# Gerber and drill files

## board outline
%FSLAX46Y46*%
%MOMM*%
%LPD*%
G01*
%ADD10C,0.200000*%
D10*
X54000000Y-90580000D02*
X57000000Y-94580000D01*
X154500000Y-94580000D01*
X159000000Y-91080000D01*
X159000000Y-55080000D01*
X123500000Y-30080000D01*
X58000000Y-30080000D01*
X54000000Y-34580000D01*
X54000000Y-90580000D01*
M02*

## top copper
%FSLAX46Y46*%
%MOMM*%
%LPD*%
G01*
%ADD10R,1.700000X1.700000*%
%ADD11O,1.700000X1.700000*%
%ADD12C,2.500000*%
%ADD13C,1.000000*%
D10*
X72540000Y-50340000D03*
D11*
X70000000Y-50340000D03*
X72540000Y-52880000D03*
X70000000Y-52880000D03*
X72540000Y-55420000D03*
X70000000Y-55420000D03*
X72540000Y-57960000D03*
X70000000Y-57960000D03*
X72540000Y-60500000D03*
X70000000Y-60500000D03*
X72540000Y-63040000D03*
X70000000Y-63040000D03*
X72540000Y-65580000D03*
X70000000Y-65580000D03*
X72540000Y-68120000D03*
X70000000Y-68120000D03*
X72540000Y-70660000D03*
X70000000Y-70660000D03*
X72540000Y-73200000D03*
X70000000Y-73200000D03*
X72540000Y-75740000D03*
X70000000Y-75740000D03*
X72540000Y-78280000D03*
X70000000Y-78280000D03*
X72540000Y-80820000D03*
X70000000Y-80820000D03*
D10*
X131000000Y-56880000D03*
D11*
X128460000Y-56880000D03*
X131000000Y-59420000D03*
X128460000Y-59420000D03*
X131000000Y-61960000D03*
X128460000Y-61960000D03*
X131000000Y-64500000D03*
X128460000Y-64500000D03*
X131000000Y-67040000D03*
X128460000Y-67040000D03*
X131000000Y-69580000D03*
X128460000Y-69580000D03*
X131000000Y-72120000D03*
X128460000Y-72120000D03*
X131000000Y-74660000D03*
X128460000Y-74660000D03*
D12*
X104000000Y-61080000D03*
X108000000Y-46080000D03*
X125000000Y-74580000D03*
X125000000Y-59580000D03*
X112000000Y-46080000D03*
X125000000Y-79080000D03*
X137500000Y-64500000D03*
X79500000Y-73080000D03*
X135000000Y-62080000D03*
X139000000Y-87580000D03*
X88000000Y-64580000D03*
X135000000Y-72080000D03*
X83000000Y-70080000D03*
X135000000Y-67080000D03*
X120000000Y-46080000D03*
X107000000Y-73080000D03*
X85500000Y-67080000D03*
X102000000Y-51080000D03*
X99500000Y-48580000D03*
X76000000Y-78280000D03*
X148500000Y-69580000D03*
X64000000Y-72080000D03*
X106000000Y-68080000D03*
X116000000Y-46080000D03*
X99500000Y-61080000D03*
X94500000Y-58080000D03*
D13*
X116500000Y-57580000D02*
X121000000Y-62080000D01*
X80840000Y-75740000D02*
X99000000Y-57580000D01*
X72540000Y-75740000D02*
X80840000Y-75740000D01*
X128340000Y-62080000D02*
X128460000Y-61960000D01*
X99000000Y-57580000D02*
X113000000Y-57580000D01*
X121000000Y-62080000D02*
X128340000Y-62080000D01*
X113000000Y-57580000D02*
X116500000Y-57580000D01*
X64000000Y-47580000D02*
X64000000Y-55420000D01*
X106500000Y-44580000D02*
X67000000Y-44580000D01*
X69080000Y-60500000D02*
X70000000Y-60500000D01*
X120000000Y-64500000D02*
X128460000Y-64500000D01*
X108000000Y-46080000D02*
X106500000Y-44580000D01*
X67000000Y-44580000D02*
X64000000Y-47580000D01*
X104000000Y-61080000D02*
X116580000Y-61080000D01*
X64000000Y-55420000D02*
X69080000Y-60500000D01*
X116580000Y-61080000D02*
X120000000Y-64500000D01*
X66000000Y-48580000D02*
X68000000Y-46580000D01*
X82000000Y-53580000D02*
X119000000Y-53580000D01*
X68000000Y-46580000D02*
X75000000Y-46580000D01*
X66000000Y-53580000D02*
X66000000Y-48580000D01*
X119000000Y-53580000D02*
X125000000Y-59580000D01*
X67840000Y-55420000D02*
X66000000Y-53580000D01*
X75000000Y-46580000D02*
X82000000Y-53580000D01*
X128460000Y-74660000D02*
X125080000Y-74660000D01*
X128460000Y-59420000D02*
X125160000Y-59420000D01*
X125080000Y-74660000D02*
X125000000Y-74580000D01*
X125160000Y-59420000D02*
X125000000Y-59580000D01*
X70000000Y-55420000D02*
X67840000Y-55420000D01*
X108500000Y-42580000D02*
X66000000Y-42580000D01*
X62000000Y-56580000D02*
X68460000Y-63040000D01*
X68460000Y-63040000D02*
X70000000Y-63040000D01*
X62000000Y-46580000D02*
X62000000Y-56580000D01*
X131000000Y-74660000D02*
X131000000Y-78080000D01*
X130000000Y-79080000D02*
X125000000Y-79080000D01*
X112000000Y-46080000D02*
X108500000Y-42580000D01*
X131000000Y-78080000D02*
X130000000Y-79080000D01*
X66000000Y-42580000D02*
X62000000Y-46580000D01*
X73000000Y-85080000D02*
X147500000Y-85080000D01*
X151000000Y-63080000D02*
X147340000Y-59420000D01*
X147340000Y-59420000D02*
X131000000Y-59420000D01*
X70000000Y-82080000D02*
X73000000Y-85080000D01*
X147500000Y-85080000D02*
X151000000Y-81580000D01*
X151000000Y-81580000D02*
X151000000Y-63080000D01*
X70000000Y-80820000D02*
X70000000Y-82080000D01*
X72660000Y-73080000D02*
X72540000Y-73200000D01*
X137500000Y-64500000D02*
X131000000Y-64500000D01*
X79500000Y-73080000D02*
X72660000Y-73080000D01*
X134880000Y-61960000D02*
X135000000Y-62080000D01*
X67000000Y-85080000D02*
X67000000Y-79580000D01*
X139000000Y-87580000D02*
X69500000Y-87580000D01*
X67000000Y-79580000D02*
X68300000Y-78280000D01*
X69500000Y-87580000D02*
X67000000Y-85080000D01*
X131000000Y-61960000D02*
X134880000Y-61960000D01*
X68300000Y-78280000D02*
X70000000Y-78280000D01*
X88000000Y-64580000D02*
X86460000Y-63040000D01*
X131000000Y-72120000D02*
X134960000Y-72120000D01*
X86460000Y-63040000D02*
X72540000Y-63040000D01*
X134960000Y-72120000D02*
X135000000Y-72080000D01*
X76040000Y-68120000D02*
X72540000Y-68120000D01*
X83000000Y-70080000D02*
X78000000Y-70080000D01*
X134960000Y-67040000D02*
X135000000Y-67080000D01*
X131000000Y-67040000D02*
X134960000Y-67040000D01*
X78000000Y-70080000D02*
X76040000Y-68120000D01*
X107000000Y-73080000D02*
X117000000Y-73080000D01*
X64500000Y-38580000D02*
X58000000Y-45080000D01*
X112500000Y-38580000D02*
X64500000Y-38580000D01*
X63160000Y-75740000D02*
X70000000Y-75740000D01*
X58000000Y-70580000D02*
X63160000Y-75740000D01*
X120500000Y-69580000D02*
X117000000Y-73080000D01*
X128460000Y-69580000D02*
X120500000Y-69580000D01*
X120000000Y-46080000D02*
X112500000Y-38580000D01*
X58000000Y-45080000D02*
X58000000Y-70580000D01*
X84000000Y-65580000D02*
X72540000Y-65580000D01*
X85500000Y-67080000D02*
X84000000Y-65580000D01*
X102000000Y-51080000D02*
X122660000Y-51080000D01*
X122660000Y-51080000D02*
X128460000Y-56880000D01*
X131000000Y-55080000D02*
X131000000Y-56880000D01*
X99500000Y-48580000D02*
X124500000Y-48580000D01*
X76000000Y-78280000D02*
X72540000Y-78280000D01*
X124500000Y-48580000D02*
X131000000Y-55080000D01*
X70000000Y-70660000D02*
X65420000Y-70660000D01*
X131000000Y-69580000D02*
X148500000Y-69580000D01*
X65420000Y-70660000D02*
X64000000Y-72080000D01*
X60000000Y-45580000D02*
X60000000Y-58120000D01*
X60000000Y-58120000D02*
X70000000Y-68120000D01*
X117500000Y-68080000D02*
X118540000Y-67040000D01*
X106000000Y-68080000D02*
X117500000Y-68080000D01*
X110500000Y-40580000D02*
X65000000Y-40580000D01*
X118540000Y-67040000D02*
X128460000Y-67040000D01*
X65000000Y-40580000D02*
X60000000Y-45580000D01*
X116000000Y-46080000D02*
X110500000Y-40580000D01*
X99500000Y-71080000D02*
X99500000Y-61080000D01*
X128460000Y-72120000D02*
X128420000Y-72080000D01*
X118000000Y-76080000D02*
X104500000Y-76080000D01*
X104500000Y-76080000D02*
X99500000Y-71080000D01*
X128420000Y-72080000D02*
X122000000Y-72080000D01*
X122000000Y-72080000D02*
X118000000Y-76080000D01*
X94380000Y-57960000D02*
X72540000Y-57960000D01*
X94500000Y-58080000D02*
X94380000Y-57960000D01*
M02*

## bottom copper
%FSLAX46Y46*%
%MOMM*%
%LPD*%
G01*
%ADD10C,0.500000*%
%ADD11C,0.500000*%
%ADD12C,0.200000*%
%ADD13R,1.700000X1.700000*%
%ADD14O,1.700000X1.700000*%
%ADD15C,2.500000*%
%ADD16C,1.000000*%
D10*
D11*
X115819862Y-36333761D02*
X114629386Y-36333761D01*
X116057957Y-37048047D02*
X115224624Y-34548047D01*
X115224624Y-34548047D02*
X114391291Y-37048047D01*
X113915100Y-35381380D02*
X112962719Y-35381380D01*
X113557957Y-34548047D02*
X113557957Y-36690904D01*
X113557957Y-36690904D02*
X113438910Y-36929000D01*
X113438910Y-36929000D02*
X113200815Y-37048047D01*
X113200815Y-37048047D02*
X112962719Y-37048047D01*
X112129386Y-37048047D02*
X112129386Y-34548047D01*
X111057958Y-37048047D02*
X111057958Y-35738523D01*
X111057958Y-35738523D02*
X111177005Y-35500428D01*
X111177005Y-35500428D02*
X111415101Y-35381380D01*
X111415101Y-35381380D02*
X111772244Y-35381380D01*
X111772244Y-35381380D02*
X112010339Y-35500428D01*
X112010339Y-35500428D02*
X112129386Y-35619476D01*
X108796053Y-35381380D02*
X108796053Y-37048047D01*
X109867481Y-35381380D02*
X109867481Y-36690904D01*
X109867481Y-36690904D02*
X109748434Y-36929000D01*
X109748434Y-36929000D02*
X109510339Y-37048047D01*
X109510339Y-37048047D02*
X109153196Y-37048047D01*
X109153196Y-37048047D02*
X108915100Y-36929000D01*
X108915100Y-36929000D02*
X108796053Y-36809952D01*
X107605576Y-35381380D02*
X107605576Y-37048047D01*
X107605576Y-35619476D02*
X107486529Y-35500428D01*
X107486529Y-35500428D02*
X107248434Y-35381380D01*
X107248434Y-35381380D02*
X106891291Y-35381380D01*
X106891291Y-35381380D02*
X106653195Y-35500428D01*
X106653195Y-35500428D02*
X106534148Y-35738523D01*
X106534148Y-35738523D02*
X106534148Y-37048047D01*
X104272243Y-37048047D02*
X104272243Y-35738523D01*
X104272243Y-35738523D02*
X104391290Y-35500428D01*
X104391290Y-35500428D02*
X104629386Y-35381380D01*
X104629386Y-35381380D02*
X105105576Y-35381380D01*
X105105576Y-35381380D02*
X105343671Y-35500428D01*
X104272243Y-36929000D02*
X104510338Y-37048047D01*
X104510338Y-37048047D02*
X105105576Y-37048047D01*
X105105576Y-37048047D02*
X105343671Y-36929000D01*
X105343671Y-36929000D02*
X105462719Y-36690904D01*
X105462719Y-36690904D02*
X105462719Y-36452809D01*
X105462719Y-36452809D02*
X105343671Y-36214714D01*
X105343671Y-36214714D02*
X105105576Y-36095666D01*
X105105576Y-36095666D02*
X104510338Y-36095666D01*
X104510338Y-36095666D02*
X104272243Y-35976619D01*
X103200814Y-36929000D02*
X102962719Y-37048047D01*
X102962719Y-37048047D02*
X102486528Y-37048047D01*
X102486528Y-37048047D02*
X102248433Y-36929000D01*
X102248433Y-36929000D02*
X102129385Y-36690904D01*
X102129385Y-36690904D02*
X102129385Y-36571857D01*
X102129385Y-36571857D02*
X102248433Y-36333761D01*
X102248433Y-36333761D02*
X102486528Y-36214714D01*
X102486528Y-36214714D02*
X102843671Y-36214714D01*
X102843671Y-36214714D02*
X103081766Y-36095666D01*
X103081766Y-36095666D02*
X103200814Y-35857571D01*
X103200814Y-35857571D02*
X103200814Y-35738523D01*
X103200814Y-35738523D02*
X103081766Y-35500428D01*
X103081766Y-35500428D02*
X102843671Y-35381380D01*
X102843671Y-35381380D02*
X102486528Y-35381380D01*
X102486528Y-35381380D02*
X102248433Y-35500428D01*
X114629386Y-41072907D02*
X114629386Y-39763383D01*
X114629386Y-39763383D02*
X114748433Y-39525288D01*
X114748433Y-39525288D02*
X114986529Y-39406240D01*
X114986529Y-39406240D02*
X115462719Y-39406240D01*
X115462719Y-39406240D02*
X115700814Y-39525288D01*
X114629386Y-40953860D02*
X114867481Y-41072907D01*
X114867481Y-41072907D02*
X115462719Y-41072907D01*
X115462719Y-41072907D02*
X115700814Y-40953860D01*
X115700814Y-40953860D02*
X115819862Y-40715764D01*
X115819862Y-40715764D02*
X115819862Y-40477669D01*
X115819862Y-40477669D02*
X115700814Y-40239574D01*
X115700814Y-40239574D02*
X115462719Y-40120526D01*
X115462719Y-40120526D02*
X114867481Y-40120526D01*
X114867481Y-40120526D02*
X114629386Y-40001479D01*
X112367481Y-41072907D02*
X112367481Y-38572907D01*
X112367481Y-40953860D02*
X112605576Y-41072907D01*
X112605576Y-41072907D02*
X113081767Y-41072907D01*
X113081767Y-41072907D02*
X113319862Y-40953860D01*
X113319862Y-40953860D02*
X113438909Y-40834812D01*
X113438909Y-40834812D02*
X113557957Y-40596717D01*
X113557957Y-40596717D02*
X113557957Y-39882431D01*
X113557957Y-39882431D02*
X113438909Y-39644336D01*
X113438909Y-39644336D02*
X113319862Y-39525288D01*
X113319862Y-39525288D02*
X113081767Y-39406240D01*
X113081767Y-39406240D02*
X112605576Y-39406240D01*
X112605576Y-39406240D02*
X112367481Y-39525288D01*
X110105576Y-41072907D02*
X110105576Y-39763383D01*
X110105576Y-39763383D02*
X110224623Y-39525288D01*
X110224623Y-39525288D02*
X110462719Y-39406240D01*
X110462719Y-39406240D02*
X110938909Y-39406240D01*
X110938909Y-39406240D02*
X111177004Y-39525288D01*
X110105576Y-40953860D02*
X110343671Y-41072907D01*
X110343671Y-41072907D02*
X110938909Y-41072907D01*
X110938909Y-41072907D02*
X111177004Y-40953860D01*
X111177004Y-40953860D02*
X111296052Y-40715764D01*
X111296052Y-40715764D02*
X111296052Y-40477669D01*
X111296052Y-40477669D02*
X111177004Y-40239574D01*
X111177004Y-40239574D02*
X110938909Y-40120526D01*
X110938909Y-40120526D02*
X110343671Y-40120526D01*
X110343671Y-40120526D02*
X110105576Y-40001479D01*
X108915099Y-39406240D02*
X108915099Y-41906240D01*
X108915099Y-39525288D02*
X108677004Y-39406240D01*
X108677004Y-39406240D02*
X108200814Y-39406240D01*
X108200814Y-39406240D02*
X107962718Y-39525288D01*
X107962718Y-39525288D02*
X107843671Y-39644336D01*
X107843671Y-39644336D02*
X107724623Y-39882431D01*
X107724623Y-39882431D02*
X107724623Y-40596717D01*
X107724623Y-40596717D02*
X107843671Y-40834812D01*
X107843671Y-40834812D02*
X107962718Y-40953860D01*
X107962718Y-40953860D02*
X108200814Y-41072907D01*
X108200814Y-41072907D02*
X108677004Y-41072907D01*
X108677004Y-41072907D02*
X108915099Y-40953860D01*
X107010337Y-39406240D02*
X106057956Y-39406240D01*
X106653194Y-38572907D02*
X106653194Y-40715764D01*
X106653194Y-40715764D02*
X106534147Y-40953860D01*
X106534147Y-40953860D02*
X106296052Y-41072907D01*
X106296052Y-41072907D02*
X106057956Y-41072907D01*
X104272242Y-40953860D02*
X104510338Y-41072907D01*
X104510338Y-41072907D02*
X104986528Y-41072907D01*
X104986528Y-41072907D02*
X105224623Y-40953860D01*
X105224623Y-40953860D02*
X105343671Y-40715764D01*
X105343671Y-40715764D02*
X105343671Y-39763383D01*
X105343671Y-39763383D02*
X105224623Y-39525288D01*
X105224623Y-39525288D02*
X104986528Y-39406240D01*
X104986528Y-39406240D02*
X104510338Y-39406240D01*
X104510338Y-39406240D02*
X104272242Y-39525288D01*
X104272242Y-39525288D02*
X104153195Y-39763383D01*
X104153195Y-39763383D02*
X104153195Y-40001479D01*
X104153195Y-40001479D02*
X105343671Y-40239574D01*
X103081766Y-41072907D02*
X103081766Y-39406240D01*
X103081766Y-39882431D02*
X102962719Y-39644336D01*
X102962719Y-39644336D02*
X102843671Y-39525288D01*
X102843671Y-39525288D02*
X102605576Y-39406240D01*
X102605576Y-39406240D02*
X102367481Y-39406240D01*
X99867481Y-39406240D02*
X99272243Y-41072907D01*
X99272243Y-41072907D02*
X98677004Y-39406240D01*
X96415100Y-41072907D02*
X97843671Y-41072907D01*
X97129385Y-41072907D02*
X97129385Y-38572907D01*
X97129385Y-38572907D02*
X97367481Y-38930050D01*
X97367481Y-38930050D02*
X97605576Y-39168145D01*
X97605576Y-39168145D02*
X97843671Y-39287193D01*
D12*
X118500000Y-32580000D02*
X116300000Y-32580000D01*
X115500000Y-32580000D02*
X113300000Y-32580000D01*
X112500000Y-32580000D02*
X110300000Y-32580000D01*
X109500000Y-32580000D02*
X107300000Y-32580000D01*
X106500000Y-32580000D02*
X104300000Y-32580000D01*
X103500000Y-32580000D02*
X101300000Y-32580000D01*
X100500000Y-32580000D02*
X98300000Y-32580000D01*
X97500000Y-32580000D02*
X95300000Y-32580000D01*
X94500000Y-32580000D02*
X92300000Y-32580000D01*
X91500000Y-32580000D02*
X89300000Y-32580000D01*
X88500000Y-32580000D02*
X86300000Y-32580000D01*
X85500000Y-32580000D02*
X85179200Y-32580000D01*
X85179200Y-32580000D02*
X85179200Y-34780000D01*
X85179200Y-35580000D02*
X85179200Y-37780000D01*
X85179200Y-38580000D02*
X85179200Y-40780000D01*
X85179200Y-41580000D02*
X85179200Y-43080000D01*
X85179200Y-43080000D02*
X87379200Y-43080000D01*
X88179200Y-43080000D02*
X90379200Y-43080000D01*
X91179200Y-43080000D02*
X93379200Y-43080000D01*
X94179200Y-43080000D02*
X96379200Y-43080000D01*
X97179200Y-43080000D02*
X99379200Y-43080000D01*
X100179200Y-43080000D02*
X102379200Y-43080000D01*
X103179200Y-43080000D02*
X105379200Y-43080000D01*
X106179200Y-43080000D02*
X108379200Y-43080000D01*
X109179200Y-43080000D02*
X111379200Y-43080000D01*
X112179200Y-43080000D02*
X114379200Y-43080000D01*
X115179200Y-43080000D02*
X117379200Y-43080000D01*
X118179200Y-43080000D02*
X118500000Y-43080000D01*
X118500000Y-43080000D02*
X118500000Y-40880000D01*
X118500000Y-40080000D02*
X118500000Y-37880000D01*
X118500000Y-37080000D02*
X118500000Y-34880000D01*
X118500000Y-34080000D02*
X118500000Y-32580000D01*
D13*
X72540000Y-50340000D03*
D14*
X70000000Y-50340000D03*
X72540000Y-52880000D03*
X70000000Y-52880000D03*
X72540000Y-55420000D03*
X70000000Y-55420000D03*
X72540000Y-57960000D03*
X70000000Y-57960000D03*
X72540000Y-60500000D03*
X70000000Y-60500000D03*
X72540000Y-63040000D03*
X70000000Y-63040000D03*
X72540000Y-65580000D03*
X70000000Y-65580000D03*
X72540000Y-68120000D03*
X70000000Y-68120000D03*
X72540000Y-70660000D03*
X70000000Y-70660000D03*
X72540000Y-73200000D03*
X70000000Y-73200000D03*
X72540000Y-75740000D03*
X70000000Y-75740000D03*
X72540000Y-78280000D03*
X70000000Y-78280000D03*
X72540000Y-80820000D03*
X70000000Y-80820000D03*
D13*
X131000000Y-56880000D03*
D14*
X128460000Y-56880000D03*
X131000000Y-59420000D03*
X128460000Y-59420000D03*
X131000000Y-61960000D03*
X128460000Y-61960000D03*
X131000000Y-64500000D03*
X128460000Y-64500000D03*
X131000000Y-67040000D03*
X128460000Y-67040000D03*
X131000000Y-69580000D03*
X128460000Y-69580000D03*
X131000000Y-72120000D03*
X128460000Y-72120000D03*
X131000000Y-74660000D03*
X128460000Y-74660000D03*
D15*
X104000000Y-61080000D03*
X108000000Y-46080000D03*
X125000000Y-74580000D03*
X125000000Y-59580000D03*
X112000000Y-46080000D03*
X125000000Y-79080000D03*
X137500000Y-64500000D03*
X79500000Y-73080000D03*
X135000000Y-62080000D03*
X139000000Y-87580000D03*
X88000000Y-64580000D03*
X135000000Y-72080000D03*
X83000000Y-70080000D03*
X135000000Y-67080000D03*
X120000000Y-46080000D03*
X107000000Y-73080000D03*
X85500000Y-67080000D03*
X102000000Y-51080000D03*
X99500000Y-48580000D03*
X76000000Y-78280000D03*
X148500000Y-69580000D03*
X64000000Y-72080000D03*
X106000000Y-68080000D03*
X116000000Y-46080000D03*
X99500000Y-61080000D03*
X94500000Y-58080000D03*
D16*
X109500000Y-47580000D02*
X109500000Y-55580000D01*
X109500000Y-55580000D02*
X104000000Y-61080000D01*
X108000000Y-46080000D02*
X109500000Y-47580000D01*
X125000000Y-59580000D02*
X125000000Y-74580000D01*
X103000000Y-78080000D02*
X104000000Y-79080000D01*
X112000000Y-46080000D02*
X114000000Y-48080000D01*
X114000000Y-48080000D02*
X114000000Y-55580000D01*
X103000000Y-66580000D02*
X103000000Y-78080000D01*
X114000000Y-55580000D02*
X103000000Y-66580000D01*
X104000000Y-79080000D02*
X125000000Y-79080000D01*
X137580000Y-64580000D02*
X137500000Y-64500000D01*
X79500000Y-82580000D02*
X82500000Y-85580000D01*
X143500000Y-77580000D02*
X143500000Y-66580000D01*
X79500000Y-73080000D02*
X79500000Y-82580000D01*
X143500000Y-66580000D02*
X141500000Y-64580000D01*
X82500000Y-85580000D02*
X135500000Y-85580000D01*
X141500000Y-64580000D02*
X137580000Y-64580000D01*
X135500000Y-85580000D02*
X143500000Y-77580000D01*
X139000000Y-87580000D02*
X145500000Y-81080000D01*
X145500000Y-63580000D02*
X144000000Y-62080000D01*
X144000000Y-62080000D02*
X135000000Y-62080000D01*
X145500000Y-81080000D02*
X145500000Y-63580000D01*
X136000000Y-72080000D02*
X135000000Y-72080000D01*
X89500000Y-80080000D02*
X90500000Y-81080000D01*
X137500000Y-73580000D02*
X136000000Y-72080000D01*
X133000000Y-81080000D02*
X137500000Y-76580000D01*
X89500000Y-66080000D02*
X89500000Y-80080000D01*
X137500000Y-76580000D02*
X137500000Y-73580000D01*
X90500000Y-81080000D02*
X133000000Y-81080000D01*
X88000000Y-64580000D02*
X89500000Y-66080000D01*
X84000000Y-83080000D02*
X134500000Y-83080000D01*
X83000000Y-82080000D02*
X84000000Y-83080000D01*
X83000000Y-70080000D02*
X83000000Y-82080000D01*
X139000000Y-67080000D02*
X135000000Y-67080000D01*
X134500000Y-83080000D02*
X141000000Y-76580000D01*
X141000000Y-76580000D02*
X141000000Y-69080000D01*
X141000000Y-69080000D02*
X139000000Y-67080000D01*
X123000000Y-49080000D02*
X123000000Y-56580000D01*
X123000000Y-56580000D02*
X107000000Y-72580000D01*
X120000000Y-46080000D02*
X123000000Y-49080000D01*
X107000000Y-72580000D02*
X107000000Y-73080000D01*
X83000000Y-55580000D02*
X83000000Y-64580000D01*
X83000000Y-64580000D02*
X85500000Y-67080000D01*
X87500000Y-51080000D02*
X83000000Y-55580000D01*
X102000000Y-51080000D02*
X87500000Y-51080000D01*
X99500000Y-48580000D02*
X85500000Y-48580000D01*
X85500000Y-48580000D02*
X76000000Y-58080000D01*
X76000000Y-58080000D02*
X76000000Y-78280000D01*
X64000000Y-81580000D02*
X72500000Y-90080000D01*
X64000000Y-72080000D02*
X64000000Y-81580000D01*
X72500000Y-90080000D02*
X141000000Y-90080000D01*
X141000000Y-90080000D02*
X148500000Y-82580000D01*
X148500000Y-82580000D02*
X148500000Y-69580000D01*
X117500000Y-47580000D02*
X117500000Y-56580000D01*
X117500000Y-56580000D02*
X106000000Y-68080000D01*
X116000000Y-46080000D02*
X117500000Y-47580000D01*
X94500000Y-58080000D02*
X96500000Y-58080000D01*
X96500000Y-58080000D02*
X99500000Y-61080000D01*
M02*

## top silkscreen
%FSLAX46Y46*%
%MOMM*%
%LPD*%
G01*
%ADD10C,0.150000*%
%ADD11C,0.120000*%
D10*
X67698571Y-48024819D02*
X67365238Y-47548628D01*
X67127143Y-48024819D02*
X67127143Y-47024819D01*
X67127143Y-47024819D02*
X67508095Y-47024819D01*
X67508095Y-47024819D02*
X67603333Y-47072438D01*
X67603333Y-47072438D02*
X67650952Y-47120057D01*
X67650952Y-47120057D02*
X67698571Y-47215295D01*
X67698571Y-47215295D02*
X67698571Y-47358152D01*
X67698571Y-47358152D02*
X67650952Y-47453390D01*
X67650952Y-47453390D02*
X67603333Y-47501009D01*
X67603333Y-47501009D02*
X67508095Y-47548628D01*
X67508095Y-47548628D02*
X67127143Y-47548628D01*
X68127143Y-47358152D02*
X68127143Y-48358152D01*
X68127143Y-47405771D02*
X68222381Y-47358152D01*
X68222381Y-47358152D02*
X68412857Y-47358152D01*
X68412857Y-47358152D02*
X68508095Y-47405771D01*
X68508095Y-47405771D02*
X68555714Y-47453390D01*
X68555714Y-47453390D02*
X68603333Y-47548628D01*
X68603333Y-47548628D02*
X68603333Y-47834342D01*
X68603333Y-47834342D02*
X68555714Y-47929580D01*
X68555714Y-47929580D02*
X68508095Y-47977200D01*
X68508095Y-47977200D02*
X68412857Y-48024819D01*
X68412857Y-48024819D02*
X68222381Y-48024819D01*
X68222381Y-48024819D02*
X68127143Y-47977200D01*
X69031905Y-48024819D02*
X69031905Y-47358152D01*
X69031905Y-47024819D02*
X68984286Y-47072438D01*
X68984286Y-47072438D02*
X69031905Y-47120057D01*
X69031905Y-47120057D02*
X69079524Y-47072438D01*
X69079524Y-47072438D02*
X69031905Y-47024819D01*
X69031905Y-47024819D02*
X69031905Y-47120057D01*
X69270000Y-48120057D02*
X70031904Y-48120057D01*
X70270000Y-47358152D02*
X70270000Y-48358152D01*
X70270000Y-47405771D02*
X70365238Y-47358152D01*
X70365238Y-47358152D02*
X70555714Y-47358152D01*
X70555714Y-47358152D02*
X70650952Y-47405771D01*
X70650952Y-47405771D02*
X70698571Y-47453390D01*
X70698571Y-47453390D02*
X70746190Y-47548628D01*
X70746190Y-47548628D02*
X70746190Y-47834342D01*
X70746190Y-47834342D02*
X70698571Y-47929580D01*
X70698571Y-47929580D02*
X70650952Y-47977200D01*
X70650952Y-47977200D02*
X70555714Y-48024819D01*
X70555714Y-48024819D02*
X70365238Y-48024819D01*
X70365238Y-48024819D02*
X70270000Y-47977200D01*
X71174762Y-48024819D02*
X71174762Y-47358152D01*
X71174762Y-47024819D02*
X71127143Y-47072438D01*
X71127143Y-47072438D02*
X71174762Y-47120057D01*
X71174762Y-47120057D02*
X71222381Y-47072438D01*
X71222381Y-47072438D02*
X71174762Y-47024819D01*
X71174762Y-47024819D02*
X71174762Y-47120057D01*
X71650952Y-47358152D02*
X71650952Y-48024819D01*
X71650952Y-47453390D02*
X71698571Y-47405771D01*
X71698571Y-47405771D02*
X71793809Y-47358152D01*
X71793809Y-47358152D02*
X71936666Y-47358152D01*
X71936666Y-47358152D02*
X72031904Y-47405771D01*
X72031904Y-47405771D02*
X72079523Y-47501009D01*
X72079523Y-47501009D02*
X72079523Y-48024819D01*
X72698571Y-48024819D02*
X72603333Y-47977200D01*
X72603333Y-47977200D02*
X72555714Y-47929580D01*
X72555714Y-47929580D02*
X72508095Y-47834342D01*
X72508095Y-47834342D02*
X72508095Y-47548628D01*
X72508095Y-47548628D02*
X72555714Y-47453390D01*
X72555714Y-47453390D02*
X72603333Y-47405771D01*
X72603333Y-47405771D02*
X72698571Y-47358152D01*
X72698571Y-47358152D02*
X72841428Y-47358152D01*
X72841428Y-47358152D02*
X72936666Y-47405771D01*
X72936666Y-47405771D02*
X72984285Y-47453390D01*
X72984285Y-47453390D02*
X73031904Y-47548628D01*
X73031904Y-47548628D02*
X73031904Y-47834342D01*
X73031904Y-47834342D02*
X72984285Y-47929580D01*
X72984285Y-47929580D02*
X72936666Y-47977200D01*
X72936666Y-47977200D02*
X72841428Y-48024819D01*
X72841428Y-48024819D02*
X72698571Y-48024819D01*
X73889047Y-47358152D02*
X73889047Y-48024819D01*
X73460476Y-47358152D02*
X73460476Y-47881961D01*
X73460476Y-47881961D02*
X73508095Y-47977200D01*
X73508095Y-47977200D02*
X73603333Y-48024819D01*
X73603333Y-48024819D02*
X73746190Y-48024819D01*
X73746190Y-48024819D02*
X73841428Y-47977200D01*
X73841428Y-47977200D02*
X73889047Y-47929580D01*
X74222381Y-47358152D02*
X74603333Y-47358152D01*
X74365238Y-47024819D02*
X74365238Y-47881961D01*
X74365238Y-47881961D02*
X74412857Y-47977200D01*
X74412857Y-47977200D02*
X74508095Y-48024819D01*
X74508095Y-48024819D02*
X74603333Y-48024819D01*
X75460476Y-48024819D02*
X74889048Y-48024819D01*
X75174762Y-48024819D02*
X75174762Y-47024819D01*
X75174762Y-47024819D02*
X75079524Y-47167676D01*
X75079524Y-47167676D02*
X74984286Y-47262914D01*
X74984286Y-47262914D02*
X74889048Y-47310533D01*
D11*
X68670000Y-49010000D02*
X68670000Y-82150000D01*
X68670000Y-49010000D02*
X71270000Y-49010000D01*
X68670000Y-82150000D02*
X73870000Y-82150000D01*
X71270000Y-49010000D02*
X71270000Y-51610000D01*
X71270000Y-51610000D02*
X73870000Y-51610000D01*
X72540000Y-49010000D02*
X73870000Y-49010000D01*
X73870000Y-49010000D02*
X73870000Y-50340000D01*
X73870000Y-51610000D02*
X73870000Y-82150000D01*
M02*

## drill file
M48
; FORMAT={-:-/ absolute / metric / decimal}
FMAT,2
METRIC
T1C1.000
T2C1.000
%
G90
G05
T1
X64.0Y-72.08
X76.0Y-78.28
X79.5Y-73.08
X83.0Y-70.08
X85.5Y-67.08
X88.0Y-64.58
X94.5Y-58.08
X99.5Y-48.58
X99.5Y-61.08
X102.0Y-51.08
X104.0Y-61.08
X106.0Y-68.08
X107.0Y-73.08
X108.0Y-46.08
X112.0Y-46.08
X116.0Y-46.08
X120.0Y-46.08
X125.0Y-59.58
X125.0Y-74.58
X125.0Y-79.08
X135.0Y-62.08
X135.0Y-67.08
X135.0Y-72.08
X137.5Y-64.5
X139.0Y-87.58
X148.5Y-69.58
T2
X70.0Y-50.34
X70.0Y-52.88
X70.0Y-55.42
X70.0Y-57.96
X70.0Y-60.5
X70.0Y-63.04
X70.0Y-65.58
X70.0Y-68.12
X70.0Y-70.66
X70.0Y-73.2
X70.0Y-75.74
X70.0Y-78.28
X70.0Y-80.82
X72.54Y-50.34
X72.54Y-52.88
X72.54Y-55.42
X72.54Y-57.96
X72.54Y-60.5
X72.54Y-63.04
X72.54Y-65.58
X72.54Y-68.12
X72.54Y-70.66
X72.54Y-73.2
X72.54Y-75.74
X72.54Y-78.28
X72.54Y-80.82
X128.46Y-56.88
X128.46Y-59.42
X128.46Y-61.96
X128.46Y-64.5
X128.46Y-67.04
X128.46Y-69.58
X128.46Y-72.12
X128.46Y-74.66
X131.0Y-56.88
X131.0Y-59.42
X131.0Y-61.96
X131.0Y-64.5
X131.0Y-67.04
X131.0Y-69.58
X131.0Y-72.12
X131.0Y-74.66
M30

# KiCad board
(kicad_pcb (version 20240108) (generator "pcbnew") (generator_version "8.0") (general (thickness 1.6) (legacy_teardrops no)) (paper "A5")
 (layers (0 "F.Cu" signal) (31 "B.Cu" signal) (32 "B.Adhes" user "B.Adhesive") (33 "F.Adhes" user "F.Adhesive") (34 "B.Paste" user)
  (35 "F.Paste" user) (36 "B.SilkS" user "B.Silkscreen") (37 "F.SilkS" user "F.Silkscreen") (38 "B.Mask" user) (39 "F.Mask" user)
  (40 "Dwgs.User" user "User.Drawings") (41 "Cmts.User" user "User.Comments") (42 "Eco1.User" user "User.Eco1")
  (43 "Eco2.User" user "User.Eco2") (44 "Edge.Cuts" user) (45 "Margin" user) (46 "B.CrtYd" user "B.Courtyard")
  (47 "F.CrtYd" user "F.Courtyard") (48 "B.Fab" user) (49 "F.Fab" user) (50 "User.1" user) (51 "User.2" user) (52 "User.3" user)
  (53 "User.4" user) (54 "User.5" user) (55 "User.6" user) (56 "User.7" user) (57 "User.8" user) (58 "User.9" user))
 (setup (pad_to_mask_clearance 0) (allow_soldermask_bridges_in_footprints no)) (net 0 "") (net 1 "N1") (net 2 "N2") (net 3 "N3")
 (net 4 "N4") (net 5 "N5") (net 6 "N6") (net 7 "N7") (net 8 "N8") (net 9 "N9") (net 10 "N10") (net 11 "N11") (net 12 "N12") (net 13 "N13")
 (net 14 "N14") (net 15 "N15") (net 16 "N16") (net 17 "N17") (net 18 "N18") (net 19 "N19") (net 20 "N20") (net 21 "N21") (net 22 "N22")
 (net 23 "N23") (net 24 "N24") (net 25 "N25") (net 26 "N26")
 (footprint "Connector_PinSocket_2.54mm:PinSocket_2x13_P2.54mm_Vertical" (layer "F.Cu") (at 72.54 50.34)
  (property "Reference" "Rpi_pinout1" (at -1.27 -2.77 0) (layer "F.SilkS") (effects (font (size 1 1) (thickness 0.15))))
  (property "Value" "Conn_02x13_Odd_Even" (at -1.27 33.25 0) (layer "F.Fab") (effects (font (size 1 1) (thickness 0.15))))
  (fp_line (start -3.87 -1.33) (end -3.87 31.81) (stroke (width 0.12) (type solid)) (layer "F.SilkS"))
  (fp_line (start -3.87 -1.33) (end -1.27 -1.33) (stroke (width 0.12) (type solid)) (layer "F.SilkS"))
  (fp_line (start -3.87 31.81) (end 1.33 31.81) (stroke (width 0.12) (type solid)) (layer "F.SilkS"))
  (fp_line (start -1.27 -1.33) (end -1.27 1.27) (stroke (width 0.12) (type solid)) (layer "F.SilkS"))
  (fp_line (start -1.27 1.27) (end 1.33 1.27) (stroke (width 0.12) (type solid)) (layer "F.SilkS"))
  (fp_line (start 0 -1.33) (end 1.33 -1.33) (stroke (width 0.12) (type solid)) (layer "F.SilkS"))
  (fp_line (start 1.33 -1.33) (end 1.33 0) (stroke (width 0.12) (type solid)) (layer "F.SilkS"))
  (fp_line (start 1.33 1.27) (end 1.33 31.81) (stroke (width 0.12) (type solid)) (layer "F.SilkS"))
  (pad "1" thru_hole rect (at 0 0) (size 1.7 1.7) (drill 1) (layers "*.Cu" "*.Mask") (remove_unused_layers no) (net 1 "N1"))
  (pad "2" thru_hole oval (at -2.54 0) (size 1.7 1.7) (drill 1) (layers "*.Cu" "*.Mask") (remove_unused_layers no) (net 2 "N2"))
  (pad "3" thru_hole oval (at 0 2.54) (size 1.7 1.7) (drill 1) (layers "*.Cu" "*.Mask") (remove_unused_layers no) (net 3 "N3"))
  (pad "4" thru_hole oval (at -2.54 2.54) (size 1.7 1.7) (drill 1) (layers "*.Cu" "*.Mask") (remove_unused_layers no) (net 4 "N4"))
  (pad "5" thru_hole oval (at 0 5.08) (size 1.7 1.7) (drill 1) (layers "*.Cu" "*.Mask") (remove_unused_layers no) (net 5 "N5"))
  (pad "6" thru_hole oval (at -2.54 5.08) (size 1.7 1.7) (drill 1) (layers "*.Cu" "*.Mask") (remove_unused_layers no) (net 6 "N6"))
  (pad "7" thru_hole oval (at 0 7.62) (size 1.7 1.7) (drill 1) (layers "*.Cu" "*.Mask") (remove_unused_layers no) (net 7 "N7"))
  (pad "8" thru_hole oval (at -2.54 7.62) (size 1.7 1.7) (drill 1) (layers "*.Cu" "*.Mask") (remove_unused_layers no) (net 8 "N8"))
  (pad "9" thru_hole oval (at 0 10.16) (size 1.7 1.7) (drill 1) (layers "*.Cu" "*.Mask") (remove_unused_layers no) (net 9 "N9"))
  (pad "10" thru_hole oval (at -2.54 10.16) (size 1.7 1.7) (drill 1) (layers "*.Cu" "*.Mask") (remove_unused_layers no) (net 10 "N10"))
  (pad "11" thru_hole oval (at 0 12.7) (size 1.7 1.7) (drill 1) (layers "*.Cu" "*.Mask") (remove_unused_layers no) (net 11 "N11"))
  (pad "12" thru_hole oval (at -2.54 12.7) (size 1.7 1.7) (drill 1) (layers "*.Cu" "*.Mask") (remove_unused_layers no) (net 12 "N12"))
  (pad "13" thru_hole oval (at 0 15.24) (size 1.7 1.7) (drill 1) (layers "*.Cu" "*.Mask") (remove_unused_layers no) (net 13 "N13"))
  (pad "14" thru_hole oval (at -2.54 15.24) (size 1.7 1.7) (drill 1) (layers "*.Cu" "*.Mask") (remove_unused_layers no) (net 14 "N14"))
  (pad "15" thru_hole oval (at 0 17.78) (size 1.7 1.7) (drill 1) (layers "*.Cu" "*.Mask") (remove_unused_layers no) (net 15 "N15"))
  (pad "16" thru_hole oval (at -2.54 17.78) (size 1.7 1.7) (drill 1) (layers "*.Cu" "*.Mask") (remove_unused_layers no) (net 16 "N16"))
  (pad "17" thru_hole oval (at 0 20.32) (size 1.7 1.7) (drill 1) (layers "*.Cu" "*.Mask") (remove_unused_layers no) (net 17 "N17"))
  (pad "18" thru_hole oval (at -2.54 20.32) (size 1.7 1.7) (drill 1) (layers "*.Cu" "*.Mask") (remove_unused_layers no) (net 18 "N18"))
  (pad "19" thru_hole oval (at 0 22.86) (size 1.7 1.7) (drill 1) (layers "*.Cu" "*.Mask") (remove_unused_layers no) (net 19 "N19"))
  (pad "20" thru_hole oval (at -2.54 22.86) (size 1.7 1.7) (drill 1) (layers "*.Cu" "*.Mask") (remove_unused_layers no) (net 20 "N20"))
  (pad "21" thru_hole oval (at 0 25.4) (size 1.7 1.7) (drill 1) (layers "*.Cu" "*.Mask") (remove_unused_layers no) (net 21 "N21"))
  (pad "22" thru_hole oval (at -2.54 25.4) (size 1.7 1.7) (drill 1) (layers "*.Cu" "*.Mask") (remove_unused_layers no) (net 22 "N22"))
  (pad "23" thru_hole oval (at 0 27.94) (size 1.7 1.7) (drill 1) (layers "*.Cu" "*.Mask") (remove_unused_layers no) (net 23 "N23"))
  (pad "24" thru_hole oval (at -2.54 27.94) (size 1.7 1.7) (drill 1) (layers "*.Cu" "*.Mask") (remove_unused_layers no) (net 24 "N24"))
  (pad "25" thru_hole oval (at 0 30.48) (size 1.7 1.7) (drill 1) (layers "*.Cu" "*.Mask") (remove_unused_layers no) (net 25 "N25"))
  (pad "26" thru_hole oval (at -2.54 30.48) (size 1.7 1.7) (drill 1) (layers "*.Cu" "*.Mask") (remove_unused_layers no) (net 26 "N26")))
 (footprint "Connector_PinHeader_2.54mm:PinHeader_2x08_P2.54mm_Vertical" (layer "B.Cu") (at 131 56.88 180)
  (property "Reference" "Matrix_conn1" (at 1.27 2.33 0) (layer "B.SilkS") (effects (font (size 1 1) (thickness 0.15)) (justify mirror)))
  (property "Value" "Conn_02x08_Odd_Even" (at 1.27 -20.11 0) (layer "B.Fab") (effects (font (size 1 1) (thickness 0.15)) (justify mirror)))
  (pad "1" thru_hole rect (at 0 0 180) (size 1.7 1.7) (drill 1) (layers "*.Cu" "*.Mask") (remove_unused_layers no) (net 23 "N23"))
  (pad "2" thru_hole oval (at 2.54 0 180) (size 1.7 1.7) (drill 1) (layers "*.Cu" "*.Mask") (remove_unused_layers no) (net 13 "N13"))
  (pad "3" thru_hole oval (at 0 -2.54 180) (size 1.7 1.7) (drill 1) (layers "*.Cu" "*.Mask") (remove_unused_layers no) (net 26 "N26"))
  (pad "4" thru_hole oval (at 2.54 -2.54 180) (size 1.7 1.7) (drill 1) (layers "*.Cu" "*.Mask") (remove_unused_layers no) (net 6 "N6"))
  (pad "5" thru_hole oval (at 0 -5.08 180) (size 1.7 1.7) (drill 1) (layers "*.Cu" "*.Mask") (remove_unused_layers no) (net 24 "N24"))
  (pad "6" thru_hole oval (at 2.54 -5.08 180) (size 1.7 1.7) (drill 1) (layers "*.Cu" "*.Mask") (remove_unused_layers no) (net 21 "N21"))
  (pad "7" thru_hole oval (at 0 -7.62 180) (size 1.7 1.7) (drill 1) (layers "*.Cu" "*.Mask") (remove_unused_layers no) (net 19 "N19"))
  (pad "8" thru_hole oval (at 2.54 -7.62 180) (size 1.7 1.7) (drill 1) (layers "*.Cu" "*.Mask") (remove_unused_layers no) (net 10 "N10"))
  (pad "9" thru_hole oval (at 0 -10.16 180) (size 1.7 1.7) (drill 1) (layers "*.Cu" "*.Mask") (remove_unused_layers no) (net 15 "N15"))
  (pad "10" thru_hole oval (at 2.54 -10.16 180) (size 1.7 1.7) (drill 1) (layers "*.Cu" "*.Mask") (remove_unused_layers no) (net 16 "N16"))
  (pad "11" thru_hole oval (at 0 -12.7 180) (size 1.7 1.7) (drill 1) (layers "*.Cu" "*.Mask") (remove_unused_layers no) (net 18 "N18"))
  (pad "12" thru_hole oval (at 2.54 -12.7 180) (size 1.7 1.7) (drill 1) (layers "*.Cu" "*.Mask") (remove_unused_layers no) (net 22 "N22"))
  (pad "13" thru_hole oval (at 0 -15.24 180) (size 1.7 1.7) (drill 1) (layers "*.Cu" "*.Mask") (remove_unused_layers no) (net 11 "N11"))
  (pad "14" thru_hole oval (at 2.54 -15.24 180) (size 1.7 1.7) (drill 1) (layers "*.Cu" "*.Mask") (remove_unused_layers no) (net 7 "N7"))
  (pad "15" thru_hole oval (at 0 -17.78 180) (size 1.7 1.7) (drill 1) (layers "*.Cu" "*.Mask") (remove_unused_layers no) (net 12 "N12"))
  (pad "16" thru_hole oval (at 2.54 -17.78 180) (size 1.7 1.7) (drill 1) (layers "*.Cu" "*.Mask") (remove_unused_layers no) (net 6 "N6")))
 (gr_poly
  (pts (xy 54 90.58) (xy 57 94.58) (xy 154.5 94.58) (xy 159 91.08) (xy 159 55.08) (xy 123.5 30.08) (xy 58 30.08) (xy 54 34.58))
  (stroke (width 0.2) (type solid)) (fill none) (layer "Edge.Cuts"))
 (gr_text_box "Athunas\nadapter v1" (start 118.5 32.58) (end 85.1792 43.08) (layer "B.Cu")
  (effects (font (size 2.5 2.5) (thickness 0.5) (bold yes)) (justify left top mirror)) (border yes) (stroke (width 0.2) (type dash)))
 (segment (start 116.5 57.58) (end 121 62.08) (width 1) (layer "F.Cu") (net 21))
 (segment (start 80.84 75.74) (end 99 57.58) (width 1) (layer "F.Cu") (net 21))
 (segment (start 72.54 75.74) (end 80.84 75.74) (width 1) (layer "F.Cu") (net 21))
 (segment (start 128.34 62.08) (end 128.46 61.96) (width 1) (layer "F.Cu") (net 21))
 (segment (start 99 57.58) (end 113 57.58) (width 1) (layer "F.Cu") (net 21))
 (segment (start 121 62.08) (end 128.34 62.08) (width 1) (layer "F.Cu") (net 21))
 (segment (start 113 57.58) (end 116.5 57.58) (width 1) (layer "F.Cu") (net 21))
 (segment (start 64 47.58) (end 64 55.42) (width 1) (layer "F.Cu") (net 10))
 (segment (start 106.5 44.58) (end 67 44.58) (width 1) (layer "F.Cu") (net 10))
 (segment (start 69.08 60.5) (end 70 60.5) (width 1) (layer "F.Cu") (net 10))
 (segment (start 120 64.5) (end 128.46 64.5) (width 1) (layer "F.Cu") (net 10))
 (segment (start 108 46.08) (end 106.5 44.58) (width 1) (layer "F.Cu") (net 10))
 (segment (start 67 44.58) (end 64 47.58) (width 1) (layer "F.Cu") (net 10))
 (segment (start 104 61.08) (end 116.58 61.08) (width 1) (layer "F.Cu") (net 10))
 (segment (start 64 55.42) (end 69.08 60.5) (width 1) (layer "F.Cu") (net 10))
 (segment (start 116.58 61.08) (end 120 64.5) (width 1) (layer "F.Cu") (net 10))
 (via (at 104 61.08) (size 2.5) (drill 1) (layers "F.Cu" "B.Cu") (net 10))
 (via (at 108 46.08) (size 2.5) (drill 1) (layers "F.Cu" "B.Cu") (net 10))
 (segment (start 109.5 47.58) (end 109.5 55.58) (width 1) (layer "B.Cu") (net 10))
 (segment (start 109.5 55.58) (end 104 61.08) (width 1) (layer "B.Cu") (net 10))
 (segment (start 108 46.08) (end 109.5 47.58) (width 1) (layer "B.Cu") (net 10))
 (segment (start 66 48.58) (end 68 46.58) (width 1) (layer "F.Cu") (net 6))
 (segment (start 82 53.58) (end 119 53.58) (width 1) (layer "F.Cu") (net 6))
 (segment (start 68 46.58) (end 75 46.58) (width 1) (layer "F.Cu") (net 6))
 (segment (start 66 53.58) (end 66 48.58) (width 1) (layer "F.Cu") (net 6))
 (segment (start 119 53.58) (end 125 59.58) (width 1) (layer "F.Cu") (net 6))
 (segment (start 67.84 55.42) (end 66 53.58) (width 1) (layer "F.Cu") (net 6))
 (segment (start 75 46.58) (end 82 53.58) (width 1) (layer "F.Cu") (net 6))
 (segment (start 128.46 74.66) (end 125.08 74.66) (width 1) (layer "F.Cu") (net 6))
 (segment (start 128.46 59.42) (end 125.16 59.42) (width 1) (layer "F.Cu") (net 6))
 (segment (start 125.08 74.66) (end 125 74.58) (width 1) (layer "F.Cu") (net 6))
 (segment (start 125.16 59.42) (end 125 59.58) (width 1) (layer "F.Cu") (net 6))
 (segment (start 70 55.42) (end 67.84 55.42) (width 1) (layer "F.Cu") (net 6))
 (via (at 125 74.58) (size 2.5) (drill 1) (layers "F.Cu" "B.Cu") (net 6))
 (via (at 125 59.58) (size 2.5) (drill 1) (layers "F.Cu" "B.Cu") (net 6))
 (segment (start 125 59.58) (end 125 74.58) (width 1) (layer "B.Cu") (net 6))
 (segment (start 108.5 42.58) (end 66 42.58) (width 1) (layer "F.Cu") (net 12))
 (segment (start 62 56.58) (end 68.46 63.04) (width 1) (layer "F.Cu") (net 12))
 (segment (start 68.46 63.04) (end 70 63.04) (width 1) (layer "F.Cu") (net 12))
 (segment (start 62 46.58) (end 62 56.58) (width 1) (layer "F.Cu") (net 12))
 (segment (start 131 74.66) (end 131 78.08) (width 1) (layer "F.Cu") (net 12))
 (segment (start 130 79.08) (end 125 79.08) (width 1) (layer "F.Cu") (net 12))
 (segment (start 112 46.08) (end 108.5 42.58) (width 1) (layer "F.Cu") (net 12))
 (segment (start 131 78.08) (end 130 79.08) (width 1) (layer "F.Cu") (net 12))
 (segment (start 66 42.58) (end 62 46.58) (width 1) (layer "F.Cu") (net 12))
 (via (at 112 46.08) (size 2.5) (drill 1) (layers "F.Cu" "B.Cu") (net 12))
 (via (at 125 79.08) (size 2.5) (drill 1) (layers "F.Cu" "B.Cu") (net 12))
 (segment (start 103 78.08) (end 104 79.08) (width 1) (layer "B.Cu") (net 12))
 (segment (start 112 46.08) (end 114 48.08) (width 1) (layer "B.Cu") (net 12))
 (segment (start 114 48.08) (end 114 55.58) (width 1) (layer "B.Cu") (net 12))
 (segment (start 103 66.58) (end 103 78.08) (width 1) (layer "B.Cu") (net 12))
 (segment (start 114 55.58) (end 103 66.58) (width 1) (layer "B.Cu") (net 12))
 (segment (start 104 79.08) (end 125 79.08) (width 1) (layer "B.Cu") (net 12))
 (segment (start 73 85.08) (end 147.5 85.08) (width 1) (layer "F.Cu") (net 26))
 (segment (start 151 63.08) (end 147.34 59.42) (width 1) (layer "F.Cu") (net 26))
 (segment (start 147.34 59.42) (end 131 59.42) (width 1) (layer "F.Cu") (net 26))
 (segment (start 70 82.08) (end 73 85.08) (width 1) (layer "F.Cu") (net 26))
 (segment (start 147.5 85.08) (end 151 81.58) (width 1) (layer "F.Cu") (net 26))
 (segment (start 151 81.58) (end 151 63.08) (width 1) (layer "F.Cu") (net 26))
 (segment (start 70 80.82) (end 70 82.08) (width 1) (layer "F.Cu") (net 26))
 (segment (start 72.66 73.08) (end 72.54 73.2) (width 1) (layer "F.Cu") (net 19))
 (segment (start 137.5 64.5) (end 131 64.5) (width 1) (layer "F.Cu") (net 19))
 (segment (start 79.5 73.08) (end 72.66 73.08) (width 1) (layer "F.Cu") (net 19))
 (via (at 137.5 64.5) (size 2.5) (drill 1) (layers "F.Cu" "B.Cu") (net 19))
 (via (at 79.5 73.08) (size 2.5) (drill 1) (layers "F.Cu" "B.Cu") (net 19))
 (segment (start 137.58 64.58) (end 137.5 64.5) (width 1) (layer "B.Cu") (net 19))
 (segment (start 79.5 82.58) (end 82.5 85.58) (width 1) (layer "B.Cu") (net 19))
 (segment (start 143.5 77.58) (end 143.5 66.58) (width 1) (layer "B.Cu") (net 19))
 (segment (start 79.5 73.08) (end 79.5 82.58) (width 1) (layer "B.Cu") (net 19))
 (segment (start 143.5 66.58) (end 141.5 64.58) (width 1) (layer "B.Cu") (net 19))
 (segment (start 82.5 85.58) (end 135.5 85.58) (width 1) (layer "B.Cu") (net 19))
 (segment (start 141.5 64.58) (end 137.58 64.58) (width 1) (layer "B.Cu") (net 19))
 (segment (start 135.5 85.58) (end 143.5 77.58) (width 1) (layer "B.Cu") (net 19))
 (segment (start 134.88 61.96) (end 135 62.08) (width 1) (layer "F.Cu") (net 24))
 (segment (start 67 85.08) (end 67 79.58) (width 1) (layer "F.Cu") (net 24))
 (segment (start 139 87.58) (end 69.5 87.58) (width 1) (layer "F.Cu") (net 24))
 (segment (start 67 79.58) (end 68.3 78.28) (width 1) (layer "F.Cu") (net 24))
 (segment (start 69.5 87.58) (end 67 85.08) (width 1) (layer "F.Cu") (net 24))
 (segment (start 131 61.96) (end 134.88 61.96) (width 1) (layer "F.Cu") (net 24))
 (segment (start 68.3 78.28) (end 70 78.28) (width 1) (layer "F.Cu") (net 24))
 (via (at 135 62.08) (size 2.5) (drill 1) (layers "F.Cu" "B.Cu") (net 24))
 (via (at 139 87.58) (size 2.5) (drill 1) (layers "F.Cu" "B.Cu") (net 24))
 (segment (start 139 87.58) (end 145.5 81.08) (width 1) (layer "B.Cu") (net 24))
 (segment (start 145.5 63.58) (end 144 62.08) (width 1) (layer "B.Cu") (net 24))
 (segment (start 144 62.08) (end 135 62.08) (width 1) (layer "B.Cu") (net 24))
 (segment (start 145.5 81.08) (end 145.5 63.58) (width 1) (layer "B.Cu") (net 24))
 (segment (start 88 64.58) (end 86.46 63.04) (width 1) (layer "F.Cu") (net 11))
 (segment (start 131 72.12) (end 134.96 72.12) (width 1) (layer "F.Cu") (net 11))
 (segment (start 86.46 63.04) (end 72.54 63.04) (width 1) (layer "F.Cu") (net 11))
 (segment (start 134.96 72.12) (end 135 72.08) (width 1) (layer "F.Cu") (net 11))
 (via (at 88 64.58) (size 2.5) (drill 1) (layers "F.Cu" "B.Cu") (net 11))
 (via (at 135 72.08) (size 2.5) (drill 1) (layers "F.Cu" "B.Cu") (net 11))
 (segment (start 136 72.08) (end 135 72.08) (width 1) (layer "B.Cu") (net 11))
 (segment (start 89.5 80.08) (end 90.5 81.08) (width 1) (layer "B.Cu") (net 11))
 (segment (start 137.5 73.58) (end 136 72.08) (width 1) (layer "B.Cu") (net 11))
 (segment (start 133 81.08) (end 137.5 76.58) (width 1) (layer "B.Cu") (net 11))
 (segment (start 89.5 66.08) (end 89.5 80.08) (width 1) (layer "B.Cu") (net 11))
 (segment (start 137.5 76.58) (end 137.5 73.58) (width 1) (layer "B.Cu") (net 11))
 (segment (start 90.5 81.08) (end 133 81.08) (width 1) (layer "B.Cu") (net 11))
 (segment (start 88 64.58) (end 89.5 66.08) (width 1) (layer "B.Cu") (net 11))
 (segment (start 76.04 68.12) (end 72.54 68.12) (width 1) (layer "F.Cu") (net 15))
 (segment (start 83 70.08) (end 78 70.08) (width 1) (layer "F.Cu") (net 15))
 (segment (start 134.96 67.04) (end 135 67.08) (width 1) (layer "F.Cu") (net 15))
 (segment (start 131 67.04) (end 134.96 67.04) (width 1) (layer "F.Cu") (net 15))
 (segment (start 78 70.08) (end 76.04 68.12) (width 1) (layer "F.Cu") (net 15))
 (via (at 83 70.08) (size 2.5) (drill 1) (layers "F.Cu" "B.Cu") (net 15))
 (via (at 135 67.08) (size 2.5) (drill 1) (layers "F.Cu" "B.Cu") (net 15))
 (segment (start 84 83.08) (end 134.5 83.08) (width 1) (layer "B.Cu") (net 15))
 (segment (start 83 82.08) (end 84 83.08) (width 1) (layer "B.Cu") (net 15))
 (segment (start 83 70.08) (end 83 82.08) (width 1) (layer "B.Cu") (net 15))
 (segment (start 139 67.08) (end 135 67.08) (width 1) (layer "B.Cu") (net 15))
 (segment (start 134.5 83.08) (end 141 76.58) (width 1) (layer "B.Cu") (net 15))
 (segment (start 141 76.58) (end 141 69.08) (width 1) (layer "B.Cu") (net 15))
 (segment (start 141 69.08) (end 139 67.08) (width 1) (layer "B.Cu") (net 15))
 (segment (start 107 73.08) (end 117 73.08) (width 1) (layer "F.Cu") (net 22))
 (segment (start 64.5 38.58) (end 58 45.08) (width 1) (layer "F.Cu") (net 22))
 (segment (start 112.5 38.58) (end 64.5 38.58) (width 1) (layer "F.Cu") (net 22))
 (segment (start 63.16 75.74) (end 70 75.74) (width 1) (layer "F.Cu") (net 22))
 (segment (start 58 70.58) (end 63.16 75.74) (width 1) (layer "F.Cu") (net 22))
 (segment (start 120.5 69.58) (end 117 73.08) (width 1) (layer "F.Cu") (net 22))
 (segment (start 128.46 69.58) (end 120.5 69.58) (width 1) (layer "F.Cu") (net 22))
 (segment (start 120 46.08) (end 112.5 38.58) (width 1) (layer "F.Cu") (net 22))
 (segment (start 58 45.08) (end 58 70.58) (width 1) (layer "F.Cu") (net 22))
 (via (at 120 46.08) (size 2.5) (drill 1) (layers "F.Cu" "B.Cu") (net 22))
 (via (at 107 73.08) (size 2.5) (drill 1) (layers "F.Cu" "B.Cu") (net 22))
 (segment (start 123 49.08) (end 123 56.58) (width 1) (layer "B.Cu") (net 22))
 (segment (start 123 56.58) (end 107 72.58) (width 1) (layer "B.Cu") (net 22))
 (segment (start 120 46.08) (end 123 49.08) (width 1) (layer "B.Cu") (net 22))
 (segment (start 107 72.58) (end 107 73.08) (width 1) (layer "B.Cu") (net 22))
 (segment (start 84 65.58) (end 72.54 65.58) (width 1) (layer "F.Cu") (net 13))
 (segment (start 85.5 67.08) (end 84 65.58) (width 1) (layer "F.Cu") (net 13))
 (segment (start 102 51.08) (end 122.66 51.08) (width 1) (layer "F.Cu") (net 13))
 (segment (start 122.66 51.08) (end 128.46 56.88) (width 1) (layer "F.Cu") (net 13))
 (via (at 85.5 67.08) (size 2.5) (drill 1) (layers "F.Cu" "B.Cu") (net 13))
 (via (at 102 51.08) (size 2.5) (drill 1) (layers "F.Cu" "B.Cu") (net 13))
 (segment (start 83 55.58) (end 83 64.58) (width 1) (layer "B.Cu") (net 13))
 (segment (start 83 64.58) (end 85.5 67.08) (width 1) (layer "B.Cu") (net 13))
 (segment (start 87.5 51.08) (end 83 55.58) (width 1) (layer "B.Cu") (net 13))
 (segment (start 102 51.08) (end 87.5 51.08) (width 1) (layer "B.Cu") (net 13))
 (segment (start 131 55.08) (end 131 56.88) (width 1) (layer "F.Cu") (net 23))
 (segment (start 99.5 48.58) (end 124.5 48.58) (width 1) (layer "F.Cu") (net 23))
 (segment (start 76 78.28) (end 72.54 78.28) (width 1) (layer "F.Cu") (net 23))
 (segment (start 124.5 48.58) (end 131 55.08) (width 1) (layer "F.Cu") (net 23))
 (via (at 99.5 48.58) (size 2.5) (drill 1) (layers "F.Cu" "B.Cu") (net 23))
 (via (at 76 78.28) (size 2.5) (drill 1) (layers "F.Cu" "B.Cu") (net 23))
 (segment (start 99.5 48.58) (end 85.5 48.58) (width 1) (layer "B.Cu") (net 23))
 (segment (start 85.5 48.58) (end 76 58.08) (width 1) (layer "B.Cu") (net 23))
 (segment (start 76 58.08) (end 76 78.28) (width 1) (layer "B.Cu") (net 23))
 (segment (start 70 70.66) (end 65.42 70.66) (width 1) (layer "F.Cu") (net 18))
 (segment (start 131 69.58) (end 148.5 69.58) (width 1) (layer "F.Cu") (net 18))
 (segment (start 65.42 70.66) (end 64 72.08) (width 1) (layer "F.Cu") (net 18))
 (via (at 148.5 69.58) (size 2.5) (drill 1) (layers "F.Cu" "B.Cu") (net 18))
 (via (at 64 72.08) (size 2.5) (drill 1) (layers "F.Cu" "B.Cu") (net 18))
 (segment (start 64 81.58) (end 72.5 90.08) (width 1) (layer "B.Cu") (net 18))
 (segment (start 64 72.08) (end 64 81.58) (width 1) (layer "B.Cu") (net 18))
 (segment (start 72.5 90.08) (end 141 90.08) (width 1) (layer "B.Cu") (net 18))
 (segment (start 141 90.08) (end 148.5 82.58) (width 1) (layer "B.Cu") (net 18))
 (segment (start 148.5 82.58) (end 148.5 69.58) (width 1) (layer "B.Cu") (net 18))
 (segment (start 60 45.58) (end 60 58.12) (width 1) (layer "F.Cu") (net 16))
 (segment (start 60 58.12) (end 70 68.12) (width 1) (layer "F.Cu") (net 16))
 (segment (start 117.5 68.08) (end 118.54 67.04) (width 1) (layer "F.Cu") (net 16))
 (segment (start 106 68.08) (end 117.5 68.08) (width 1) (layer "F.Cu") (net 16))
 (segment (start 110.5 40.58) (end 65 40.58) (width 1) (layer "F.Cu") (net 16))
 (segment (start 118.54 67.04) (end 128.46 67.04) (width 1) (layer "F.Cu") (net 16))
 (segment (start 65 40.58) (end 60 45.58) (width 1) (layer "F.Cu") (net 16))
 (segment (start 116 46.08) (end 110.5 40.58) (width 1) (layer "F.Cu") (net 16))
 (via (at 106 68.08) (size 2.5) (drill 1) (layers "F.Cu" "B.Cu") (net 16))
 (via (at 116 46.08) (size 2.5) (drill 1) (layers "F.Cu" "B.Cu") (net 16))
 (segment (start 117.5 47.58) (end 117.5 56.58) (width 1) (layer "B.Cu") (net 16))
 (segment (start 117.5 56.58) (end 106 68.08) (width 1) (layer "B.Cu") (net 16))
 (segment (start 116 46.08) (end 117.5 47.58) (width 1) (layer "B.Cu") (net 16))
 (segment (start 99.5 71.08) (end 99.5 61.08) (width 1) (layer "F.Cu") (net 7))
 (segment (start 128.46 72.12) (end 128.42 72.08) (width 1) (layer "F.Cu") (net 7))
 (segment (start 118 76.08) (end 104.5 76.08) (width 1) (layer "F.Cu") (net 7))
 (segment (start 104.5 76.08) (end 99.5 71.08) (width 1) (layer "F.Cu") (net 7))
 (segment (start 128.42 72.08) (end 122 72.08) (width 1) (layer "F.Cu") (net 7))
 (segment (start 122 72.08) (end 118 76.08) (width 1) (layer "F.Cu") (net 7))
 (segment (start 94.38 57.96) (end 72.54 57.96) (width 1) (layer "F.Cu") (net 7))
 (segment (start 94.5 58.08) (end 94.38 57.96) (width 1) (layer "F.Cu") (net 7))
 (via (at 99.5 61.08) (size 2.5) (drill 1) (layers "F.Cu" "B.Cu") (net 7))
 (via (at 94.5 58.08) (size 2.5) (drill 1) (layers "F.Cu" "B.Cu") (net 7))
 (segment (start 94.5 58.08) (end 96.5 58.08) (width 1) (layer "B.Cu") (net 7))
 (segment (start 96.5 58.08) (end 99.5 61.08) (width 1) (layer "B.Cu") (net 7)))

